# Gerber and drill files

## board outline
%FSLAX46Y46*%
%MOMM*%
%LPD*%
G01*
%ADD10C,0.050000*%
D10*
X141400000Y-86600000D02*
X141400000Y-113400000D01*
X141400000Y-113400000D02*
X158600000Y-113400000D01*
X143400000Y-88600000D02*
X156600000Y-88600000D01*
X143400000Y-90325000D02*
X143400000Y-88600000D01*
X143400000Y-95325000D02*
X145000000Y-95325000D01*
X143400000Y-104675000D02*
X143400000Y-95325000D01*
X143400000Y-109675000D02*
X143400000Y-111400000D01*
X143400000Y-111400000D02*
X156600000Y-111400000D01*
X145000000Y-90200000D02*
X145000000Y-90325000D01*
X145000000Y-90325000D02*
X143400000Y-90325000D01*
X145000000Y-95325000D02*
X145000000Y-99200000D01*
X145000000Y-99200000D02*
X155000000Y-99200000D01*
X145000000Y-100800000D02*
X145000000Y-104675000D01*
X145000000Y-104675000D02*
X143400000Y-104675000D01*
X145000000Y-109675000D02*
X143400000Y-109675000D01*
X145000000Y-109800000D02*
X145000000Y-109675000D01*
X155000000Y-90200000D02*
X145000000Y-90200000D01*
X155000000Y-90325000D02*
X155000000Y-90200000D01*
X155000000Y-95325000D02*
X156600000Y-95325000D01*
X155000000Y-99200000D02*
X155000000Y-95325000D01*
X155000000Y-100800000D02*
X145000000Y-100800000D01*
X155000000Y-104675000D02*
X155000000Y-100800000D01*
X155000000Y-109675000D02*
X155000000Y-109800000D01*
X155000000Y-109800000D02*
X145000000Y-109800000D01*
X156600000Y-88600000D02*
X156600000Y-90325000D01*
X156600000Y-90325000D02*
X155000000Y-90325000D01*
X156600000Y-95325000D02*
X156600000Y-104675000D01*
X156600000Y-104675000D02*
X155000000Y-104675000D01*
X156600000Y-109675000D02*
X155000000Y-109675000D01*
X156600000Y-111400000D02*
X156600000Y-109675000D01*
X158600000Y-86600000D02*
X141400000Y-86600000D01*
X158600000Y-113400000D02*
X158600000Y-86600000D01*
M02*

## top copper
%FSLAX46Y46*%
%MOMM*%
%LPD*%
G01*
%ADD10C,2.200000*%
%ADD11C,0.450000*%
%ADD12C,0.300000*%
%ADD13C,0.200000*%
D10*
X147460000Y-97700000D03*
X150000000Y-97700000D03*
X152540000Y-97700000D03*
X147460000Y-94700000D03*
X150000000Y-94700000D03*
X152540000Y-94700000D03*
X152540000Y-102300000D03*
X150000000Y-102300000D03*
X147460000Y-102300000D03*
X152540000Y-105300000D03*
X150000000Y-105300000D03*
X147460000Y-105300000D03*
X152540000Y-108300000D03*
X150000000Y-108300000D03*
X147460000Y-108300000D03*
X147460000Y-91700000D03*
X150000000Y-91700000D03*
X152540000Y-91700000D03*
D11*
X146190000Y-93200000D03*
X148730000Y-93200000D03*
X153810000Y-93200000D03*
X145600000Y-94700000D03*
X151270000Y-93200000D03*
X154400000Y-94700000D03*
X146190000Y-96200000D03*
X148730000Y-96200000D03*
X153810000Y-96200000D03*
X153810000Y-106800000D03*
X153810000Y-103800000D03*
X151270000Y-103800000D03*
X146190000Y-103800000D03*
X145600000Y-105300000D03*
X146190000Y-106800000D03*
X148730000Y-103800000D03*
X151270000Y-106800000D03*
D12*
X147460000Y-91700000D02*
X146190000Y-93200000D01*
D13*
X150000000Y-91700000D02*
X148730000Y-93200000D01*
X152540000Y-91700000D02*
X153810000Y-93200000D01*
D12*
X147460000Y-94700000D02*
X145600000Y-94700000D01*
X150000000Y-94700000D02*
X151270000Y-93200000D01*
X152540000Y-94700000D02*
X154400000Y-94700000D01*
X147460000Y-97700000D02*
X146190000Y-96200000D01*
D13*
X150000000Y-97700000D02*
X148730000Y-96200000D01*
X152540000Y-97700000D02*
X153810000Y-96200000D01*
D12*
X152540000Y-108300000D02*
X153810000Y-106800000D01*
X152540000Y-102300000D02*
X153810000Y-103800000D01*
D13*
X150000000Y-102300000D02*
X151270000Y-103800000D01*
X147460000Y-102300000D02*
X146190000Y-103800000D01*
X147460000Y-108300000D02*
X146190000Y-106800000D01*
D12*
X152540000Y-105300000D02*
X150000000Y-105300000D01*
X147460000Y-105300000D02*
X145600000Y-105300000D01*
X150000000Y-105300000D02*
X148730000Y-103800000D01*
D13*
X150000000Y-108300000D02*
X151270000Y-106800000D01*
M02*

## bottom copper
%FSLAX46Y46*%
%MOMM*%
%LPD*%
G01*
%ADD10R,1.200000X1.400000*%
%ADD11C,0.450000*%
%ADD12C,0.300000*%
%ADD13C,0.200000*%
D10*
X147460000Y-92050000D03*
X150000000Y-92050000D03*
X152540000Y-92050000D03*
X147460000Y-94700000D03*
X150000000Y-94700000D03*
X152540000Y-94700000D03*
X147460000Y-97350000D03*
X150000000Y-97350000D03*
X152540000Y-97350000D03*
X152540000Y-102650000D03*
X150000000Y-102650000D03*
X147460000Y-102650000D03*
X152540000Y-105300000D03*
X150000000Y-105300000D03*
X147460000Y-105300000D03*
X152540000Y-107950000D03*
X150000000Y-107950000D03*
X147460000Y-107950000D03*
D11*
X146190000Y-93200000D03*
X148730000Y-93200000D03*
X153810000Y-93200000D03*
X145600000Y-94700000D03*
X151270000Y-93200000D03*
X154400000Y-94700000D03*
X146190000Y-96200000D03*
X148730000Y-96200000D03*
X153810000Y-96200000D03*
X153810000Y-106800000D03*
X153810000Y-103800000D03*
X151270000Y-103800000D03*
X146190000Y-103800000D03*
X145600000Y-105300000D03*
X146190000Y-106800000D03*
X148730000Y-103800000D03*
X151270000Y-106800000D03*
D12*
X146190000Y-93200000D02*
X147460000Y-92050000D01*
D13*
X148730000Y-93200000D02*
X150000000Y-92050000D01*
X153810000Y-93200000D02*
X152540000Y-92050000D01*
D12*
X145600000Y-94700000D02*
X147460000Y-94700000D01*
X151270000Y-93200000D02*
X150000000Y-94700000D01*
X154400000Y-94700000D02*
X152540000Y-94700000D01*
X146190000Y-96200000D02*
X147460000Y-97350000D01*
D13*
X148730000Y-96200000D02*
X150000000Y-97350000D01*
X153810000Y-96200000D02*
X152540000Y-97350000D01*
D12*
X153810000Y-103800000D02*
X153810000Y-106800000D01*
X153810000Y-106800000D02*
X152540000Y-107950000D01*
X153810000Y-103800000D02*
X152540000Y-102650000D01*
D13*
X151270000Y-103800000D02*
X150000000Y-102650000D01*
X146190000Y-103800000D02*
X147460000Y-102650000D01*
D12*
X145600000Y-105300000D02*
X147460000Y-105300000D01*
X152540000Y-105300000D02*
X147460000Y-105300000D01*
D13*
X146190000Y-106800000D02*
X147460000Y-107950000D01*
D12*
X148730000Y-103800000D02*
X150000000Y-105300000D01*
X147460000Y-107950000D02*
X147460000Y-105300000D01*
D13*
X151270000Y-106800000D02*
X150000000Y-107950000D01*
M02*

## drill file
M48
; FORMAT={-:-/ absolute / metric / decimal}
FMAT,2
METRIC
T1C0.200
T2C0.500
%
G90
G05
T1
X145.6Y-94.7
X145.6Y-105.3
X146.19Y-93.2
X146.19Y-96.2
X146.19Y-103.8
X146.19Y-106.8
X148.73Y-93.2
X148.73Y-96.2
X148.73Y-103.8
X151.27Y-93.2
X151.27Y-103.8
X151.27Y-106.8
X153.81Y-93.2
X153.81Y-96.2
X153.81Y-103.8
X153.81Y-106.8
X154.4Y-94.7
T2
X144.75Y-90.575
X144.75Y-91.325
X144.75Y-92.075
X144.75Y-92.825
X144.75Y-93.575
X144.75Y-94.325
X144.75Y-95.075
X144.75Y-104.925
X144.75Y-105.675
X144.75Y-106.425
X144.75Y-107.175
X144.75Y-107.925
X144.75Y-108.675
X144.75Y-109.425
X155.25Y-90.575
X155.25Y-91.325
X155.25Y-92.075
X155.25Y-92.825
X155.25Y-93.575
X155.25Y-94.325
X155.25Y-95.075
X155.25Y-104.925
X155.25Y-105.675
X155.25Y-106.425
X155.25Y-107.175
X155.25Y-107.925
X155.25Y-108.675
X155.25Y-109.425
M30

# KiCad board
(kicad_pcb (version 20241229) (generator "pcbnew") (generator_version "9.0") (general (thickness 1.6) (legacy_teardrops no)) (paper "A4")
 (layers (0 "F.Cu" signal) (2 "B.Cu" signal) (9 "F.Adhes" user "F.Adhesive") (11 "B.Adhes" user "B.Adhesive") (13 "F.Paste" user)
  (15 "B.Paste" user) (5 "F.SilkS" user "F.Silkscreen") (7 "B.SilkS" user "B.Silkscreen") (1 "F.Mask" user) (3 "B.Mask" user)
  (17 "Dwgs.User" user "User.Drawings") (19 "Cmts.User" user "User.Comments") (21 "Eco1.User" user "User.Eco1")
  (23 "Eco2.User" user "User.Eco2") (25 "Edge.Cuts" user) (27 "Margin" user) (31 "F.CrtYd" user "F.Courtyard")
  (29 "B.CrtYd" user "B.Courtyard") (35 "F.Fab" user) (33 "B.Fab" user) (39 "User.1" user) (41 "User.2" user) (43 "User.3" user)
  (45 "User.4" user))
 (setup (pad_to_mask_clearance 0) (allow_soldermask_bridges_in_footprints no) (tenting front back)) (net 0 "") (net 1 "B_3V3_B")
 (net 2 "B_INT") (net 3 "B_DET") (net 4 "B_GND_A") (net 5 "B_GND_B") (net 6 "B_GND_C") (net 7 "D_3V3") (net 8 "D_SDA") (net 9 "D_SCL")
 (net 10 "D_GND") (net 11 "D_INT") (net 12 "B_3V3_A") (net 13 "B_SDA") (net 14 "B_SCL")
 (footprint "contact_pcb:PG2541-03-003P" (layer "F.Cu") (at 150 97.7)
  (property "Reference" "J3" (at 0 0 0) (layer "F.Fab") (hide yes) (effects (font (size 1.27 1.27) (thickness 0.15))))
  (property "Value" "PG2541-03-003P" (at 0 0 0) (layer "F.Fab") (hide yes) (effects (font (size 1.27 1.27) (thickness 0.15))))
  (pad "1" smd circle (at -2.54 0) (size 2.2 2.2) (layers "F.Cu" "F.Mask" "F.Paste") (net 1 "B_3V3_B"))
  (pad "2" smd circle (at 0 0) (size 2.2 2.2) (layers "F.Cu" "F.Mask" "F.Paste") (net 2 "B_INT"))
  (pad "3" smd circle (at 2.54 0) (size 2.2 2.2) (layers "F.Cu" "F.Mask" "F.Paste") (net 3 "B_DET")))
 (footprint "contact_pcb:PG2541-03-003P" (layer "F.Cu") (at 150 94.7)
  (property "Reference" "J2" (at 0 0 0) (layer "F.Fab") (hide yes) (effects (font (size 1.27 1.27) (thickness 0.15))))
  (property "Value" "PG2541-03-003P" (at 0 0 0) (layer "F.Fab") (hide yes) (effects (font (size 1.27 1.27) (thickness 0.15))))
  (pad "1" smd circle (at -2.54 0) (size 2.2 2.2) (layers "F.Cu" "F.Mask" "F.Paste") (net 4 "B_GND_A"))
  (pad "2" smd circle (at 0 0) (size 2.2 2.2) (layers "F.Cu" "F.Mask" "F.Paste") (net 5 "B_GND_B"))
  (pad "3" smd circle (at 2.54 0) (size 2.2 2.2) (layers "F.Cu" "F.Mask" "F.Paste") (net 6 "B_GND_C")))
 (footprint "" (layer "F.Cu") (at 150 105.3)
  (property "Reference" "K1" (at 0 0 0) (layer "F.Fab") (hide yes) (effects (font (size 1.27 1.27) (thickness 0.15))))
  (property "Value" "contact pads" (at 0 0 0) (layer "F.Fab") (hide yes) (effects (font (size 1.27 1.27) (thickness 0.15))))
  (pad "1" smd circle (at 2.54 -3) (size 2.2 2.2) (layers "F.Cu" "F.Mask") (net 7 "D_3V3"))
  (pad "2" smd circle (at 0 -3) (size 2.2 2.2) (layers "F.Cu" "F.Mask") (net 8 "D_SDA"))
  (pad "3" smd circle (at -2.54 -3) (size 2.2 2.2) (layers "F.Cu" "F.Mask") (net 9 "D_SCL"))
  (pad "4" smd circle (at 2.54 0) (size 2.2 2.2) (layers "F.Cu" "F.Mask") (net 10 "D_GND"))
  (pad "5" smd circle (at 0 0) (size 2.2 2.2) (layers "F.Cu" "F.Mask") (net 10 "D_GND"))
  (pad "6" smd circle (at -2.54 0) (size 2.2 2.2) (layers "F.Cu" "F.Mask") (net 10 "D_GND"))
  (pad "7" smd circle (at 2.54 3) (size 2.2 2.2) (layers "F.Cu" "F.Mask") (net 7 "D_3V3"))
  (pad "8" smd circle (at 0 3) (size 2.2 2.2) (layers "F.Cu" "F.Mask") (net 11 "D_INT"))
  (pad "9" smd circle (at -2.54 3) (size 2.2 2.2) (layers "F.Cu" "F.Mask") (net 10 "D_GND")))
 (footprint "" (layer "F.Cu") (at 150 94.7)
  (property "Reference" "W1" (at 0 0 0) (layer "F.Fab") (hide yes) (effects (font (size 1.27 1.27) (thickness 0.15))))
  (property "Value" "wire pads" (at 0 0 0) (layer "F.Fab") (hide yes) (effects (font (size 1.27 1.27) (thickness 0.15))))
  (pad "1" smd rect (at -2.54 -2.65) (size 1.2 1.4) (layers "B.Cu" "B.Mask") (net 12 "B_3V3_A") (thermal_bridge_angle 45))
  (pad "2" smd rect (at 0 -2.65) (size 1.2 1.4) (layers "B.Cu" "B.Mask") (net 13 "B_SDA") (thermal_bridge_angle 45))
  (pad "3" smd rect (at 2.54 -2.65) (size 1.2 1.4) (layers "B.Cu" "B.Mask") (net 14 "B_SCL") (thermal_bridge_angle 45))
  (pad "4" smd rect (at -2.54 0) (size 1.2 1.4) (layers "B.Cu" "B.Mask") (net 4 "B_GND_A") (thermal_bridge_angle 45))
  (pad "5" smd rect (at 0 0) (size 1.2 1.4) (layers "B.Cu" "B.Mask") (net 5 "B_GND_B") (thermal_bridge_angle 45))
  (pad "6" smd rect (at 2.54 0) (size 1.2 1.4) (layers "B.Cu" "B.Mask") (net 6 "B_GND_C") (thermal_bridge_angle 45))
  (pad "7" smd rect (at -2.54 2.65) (size 1.2 1.4) (layers "B.Cu" "B.Mask") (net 1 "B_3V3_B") (thermal_bridge_angle 45))
  (pad "8" smd rect (at 0 2.65) (size 1.2 1.4) (layers "B.Cu" "B.Mask") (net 2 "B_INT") (thermal_bridge_angle 45))
  (pad "9" smd rect (at 2.54 2.65) (size 1.2 1.4) (layers "B.Cu" "B.Mask") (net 3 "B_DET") (thermal_bridge_angle 45)))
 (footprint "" (layer "F.Cu") (at 150 105.3)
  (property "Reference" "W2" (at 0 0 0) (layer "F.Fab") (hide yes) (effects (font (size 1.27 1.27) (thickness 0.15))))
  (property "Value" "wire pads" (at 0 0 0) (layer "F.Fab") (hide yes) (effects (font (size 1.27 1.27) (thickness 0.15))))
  (pad "1" smd rect (at 2.54 -2.65) (size 1.2 1.4) (layers "B.Cu" "B.Mask") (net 7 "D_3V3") (thermal_bridge_angle 45))
  (pad "2" smd rect (at 0 -2.65) (size 1.2 1.4) (layers "B.Cu" "B.Mask") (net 8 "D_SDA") (thermal_bridge_angle 45))
  (pad "3" smd rect (at -2.54 -2.65) (size 1.2 1.4) (layers "B.Cu" "B.Mask") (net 9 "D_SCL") (thermal_bridge_angle 45))
  (pad "4" smd rect (at 2.54 0) (size 1.2 1.4) (layers "B.Cu" "B.Mask") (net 10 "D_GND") (thermal_bridge_angle 45))
  (pad "5" smd rect (at 0 0) (size 1.2 1.4) (layers "B.Cu" "B.Mask") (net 10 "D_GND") (thermal_bridge_angle 45))
  (pad "6" smd rect (at -2.54 0) (size 1.2 1.4) (layers "B.Cu" "B.Mask") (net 10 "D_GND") (thermal_bridge_angle 45))
  (pad "7" smd rect (at 2.54 2.65) (size 1.2 1.4) (layers "B.Cu" "B.Mask") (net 7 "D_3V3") (thermal_bridge_angle 45))
  (pad "8" smd rect (at 0 2.65) (size 1.2 1.4) (layers "B.Cu" "B.Mask") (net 11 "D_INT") (thermal_bridge_angle 45))
  (pad "9" smd rect (at -2.54 2.65) (size 1.2 1.4) (layers "B.Cu" "B.Mask") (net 10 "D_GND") (thermal_bridge_angle 45)))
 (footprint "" (layer "F.Cu") (at 150 100)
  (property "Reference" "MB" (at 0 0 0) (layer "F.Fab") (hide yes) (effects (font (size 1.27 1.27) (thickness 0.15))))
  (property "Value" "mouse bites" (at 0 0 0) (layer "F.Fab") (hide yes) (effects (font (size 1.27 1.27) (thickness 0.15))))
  (pad "" np_thru_hole circle (at -5.25 -9.425) (size 0.5 0.5) (drill 0.5) (layers "*.Mask"))
  (pad "" np_thru_hole circle (at -5.25 -8.675) (size 0.5 0.5) (drill 0.5) (layers "*.Mask"))
  (pad "" np_thru_hole circle (at -5.25 -7.925) (size 0.5 0.5) (drill 0.5) (layers "*.Mask"))
  (pad "" np_thru_hole circle (at -5.25 -7.175) (size 0.5 0.5) (drill 0.5) (layers "*.Mask"))
  (pad "" np_thru_hole circle (at -5.25 -6.425) (size 0.5 0.5) (drill 0.5) (layers "*.Mask"))
  (pad "" np_thru_hole circle (at -5.25 -5.675) (size 0.5 0.5) (drill 0.5) (layers "*.Mask"))
  (pad "" np_thru_hole circle (at -5.25 -4.925) (size 0.5 0.5) (drill 0.5) (layers "*.Mask"))
  (pad "" np_thru_hole circle (at -5.25 4.925) (size 0.5 0.5) (drill 0.5) (layers "*.Mask"))
  (pad "" np_thru_hole circle (at -5.25 5.675) (size 0.5 0.5) (drill 0.5) (layers "*.Mask"))
  (pad "" np_thru_hole circle (at -5.25 6.425) (size 0.5 0.5) (drill 0.5) (layers "*.Mask"))
  (pad "" np_thru_hole circle (at -5.25 7.175) (size 0.5 0.5) (drill 0.5) (layers "*.Mask"))
  (pad "" np_thru_hole circle (at -5.25 7.925) (size 0.5 0.5) (drill 0.5) (layers "*.Mask"))
  (pad "" np_thru_hole circle (at -5.25 8.675) (size 0.5 0.5) (drill 0.5) (layers "*.Mask"))
  (pad "" np_thru_hole circle (at -5.25 9.425) (size 0.5 0.5) (drill 0.5) (layers "*.Mask"))
  (pad "" np_thru_hole circle (at 5.25 -9.425) (size 0.5 0.5) (drill 0.5) (layers "*.Mask"))
  (pad "" np_thru_hole circle (at 5.25 -8.675) (size 0.5 0.5) (drill 0.5) (layers "*.Mask"))
  (pad "" np_thru_hole circle (at 5.25 -7.925) (size 0.5 0.5) (drill 0.5) (layers "*.Mask"))
  (pad "" np_thru_hole circle (at 5.25 -7.175) (size 0.5 0.5) (drill 0.5) (layers "*.Mask"))
  (pad "" np_thru_hole circle (at 5.25 -6.425) (size 0.5 0.5) (drill 0.5) (layers "*.Mask"))
  (pad "" np_thru_hole circle (at 5.25 -5.675) (size 0.5 0.5) (drill 0.5) (layers "*.Mask"))
  (pad "" np_thru_hole circle (at 5.25 -4.925) (size 0.5 0.5) (drill 0.5) (layers "*.Mask"))
  (pad "" np_thru_hole circle (at 5.25 4.925) (size 0.5 0.5) (drill 0.5) (layers "*.Mask"))
  (pad "" np_thru_hole circle (at 5.25 5.675) (size 0.5 0.5) (drill 0.5) (layers "*.Mask"))
  (pad "" np_thru_hole circle (at 5.25 6.425) (size 0.5 0.5) (drill 0.5) (layers "*.Mask"))
  (pad "" np_thru_hole circle (at 5.25 7.175) (size 0.5 0.5) (drill 0.5) (layers "*.Mask"))
  (pad "" np_thru_hole circle (at 5.25 7.925) (size 0.5 0.5) (drill 0.5) (layers "*.Mask"))
  (pad "" np_thru_hole circle (at 5.25 8.675) (size 0.5 0.5) (drill 0.5) (layers "*.Mask"))
  (pad "" np_thru_hole circle (at 5.25 9.425) (size 0.5 0.5) (drill 0.5) (layers "*.Mask")))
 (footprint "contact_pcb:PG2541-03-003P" (layer "F.Cu") (at 150 91.7)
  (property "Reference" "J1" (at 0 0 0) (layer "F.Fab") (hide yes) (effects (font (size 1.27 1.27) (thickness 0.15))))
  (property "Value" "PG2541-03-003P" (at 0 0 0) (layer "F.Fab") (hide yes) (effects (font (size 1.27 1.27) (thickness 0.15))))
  (pad "1" smd circle (at -2.54 0) (size 2.2 2.2) (layers "F.Cu" "F.Mask" "F.Paste") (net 12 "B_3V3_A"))
  (pad "2" smd circle (at 0 0) (size 2.2 2.2) (layers "F.Cu" "F.Mask" "F.Paste") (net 13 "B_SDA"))
  (pad "3" smd circle (at 2.54 0) (size 2.2 2.2) (layers "F.Cu" "F.Mask" "F.Paste") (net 14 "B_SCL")))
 (gr_line (start 141.4 86.6) (end 141.4 113.4) (stroke (width 0.05) (type default)) (layer "Edge.Cuts"))
 (gr_line (start 141.4 113.4) (end 158.6 113.4) (stroke (width 0.05) (type default)) (layer "Edge.Cuts"))
 (gr_line (start 143.4 88.6) (end 156.6 88.6) (stroke (width 0.05) (type default)) (layer "Edge.Cuts"))
 (gr_line (start 143.4 90.325) (end 143.4 88.6) (stroke (width 0.05) (type default)) (layer "Edge.Cuts"))
 (gr_line (start 143.4 95.325) (end 145 95.325) (stroke (width 0.05) (type default)) (layer "Edge.Cuts"))
 (gr_line (start 143.4 104.675) (end 143.4 95.325) (stroke (width 0.05) (type default)) (layer "Edge.Cuts"))
 (gr_line (start 143.4 109.675) (end 143.4 111.4) (stroke (width 0.05) (type default)) (layer "Edge.Cuts"))
 (gr_line (start 143.4 111.4) (end 156.6 111.4) (stroke (width 0.05) (type default)) (layer "Edge.Cuts"))
 (gr_line (start 145 90.2) (end 145 90.325) (stroke (width 0.05) (type default)) (layer "Edge.Cuts"))
 (gr_line (start 145 90.325) (end 143.4 90.325) (stroke (width 0.05) (type default)) (layer "Edge.Cuts"))
 (gr_line (start 145 95.325) (end 145 99.2) (stroke (width 0.05) (type default)) (layer "Edge.Cuts"))
 (gr_line (start 145 99.2) (end 155 99.2) (stroke (width 0.05) (type default)) (layer "Edge.Cuts"))
 (gr_line (start 145 100.8) (end 145 104.675) (stroke (width 0.05) (type default)) (layer "Edge.Cuts"))
 (gr_line (start 145 104.675) (end 143.4 104.675) (stroke (width 0.05) (type default)) (layer "Edge.Cuts"))
 (gr_line (start 145 109.675) (end 143.4 109.675) (stroke (width 0.05) (type default)) (layer "Edge.Cuts"))
 (gr_line (start 145 109.8) (end 145 109.675) (stroke (width 0.05) (type default)) (layer "Edge.Cuts"))
 (gr_line (start 155 90.2) (end 145 90.2) (stroke (width 0.05) (type default)) (layer "Edge.Cuts"))
 (gr_line (start 155 90.325) (end 155 90.2) (stroke (width 0.05) (type default)) (layer "Edge.Cuts"))
 (gr_line (start 155 95.325) (end 156.6 95.325) (stroke (width 0.05) (type default)) (layer "Edge.Cuts"))
 (gr_line (start 155 99.2) (end 155 95.325) (stroke (width 0.05) (type default)) (layer "Edge.Cuts"))
 (gr_line (start 155 100.8) (end 145 100.8) (stroke (width 0.05) (type default)) (layer "Edge.Cuts"))
 (gr_line (start 155 104.675) (end 155 100.8) (stroke (width 0.05) (type default)) (layer "Edge.Cuts"))
 (gr_line (start 155 109.675) (end 155 109.8) (stroke (width 0.05) (type default)) (layer "Edge.Cuts"))
 (gr_line (start 155 109.8) (end 145 109.8) (stroke (width 0.05) (type default)) (layer "Edge.Cuts"))
 (gr_line (start 156.6 88.6) (end 156.6 90.325) (stroke (width 0.05) (type default)) (layer "Edge.Cuts"))
 (gr_line (start 156.6 90.325) (end 155 90.325) (stroke (width 0.05) (type default)) (layer "Edge.Cuts"))
 (gr_line (start 156.6 95.325) (end 156.6 104.675) (stroke (width 0.05) (type default)) (layer "Edge.Cuts"))
 (gr_line (start 156.6 104.675) (end 155 104.675) (stroke (width 0.05) (type default)) (layer "Edge.Cuts"))
 (gr_line (start 156.6 109.675) (end 155 109.675) (stroke (width 0.05) (type default)) (layer "Edge.Cuts"))
 (gr_line (start 156.6 111.4) (end 156.6 109.675) (stroke (width 0.05) (type default)) (layer "Edge.Cuts"))
 (gr_line (start 158.6 86.6) (end 141.4 86.6) (stroke (width 0.05) (type default)) (layer "Edge.Cuts"))
 (gr_line (start 158.6 113.4) (end 158.6 86.6) (stroke (width 0.05) (type default)) (layer "Edge.Cuts"))
 (segment (start 147.46 91.7) (end 146.19 93.2) (width 0.3) (layer "F.Cu") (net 12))
 (via (at 146.19 93.2) (size 0.45) (drill 0.2) (layers "F.Cu" "B.Cu") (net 12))
 (segment (start 146.19 93.2) (end 147.46 92.05) (width 0.3) (layer "B.Cu") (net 12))
 (segment (start 150 91.7) (end 148.73 93.2) (width 0.2) (layer "F.Cu") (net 13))
 (via (at 148.73 93.2) (size 0.45) (drill 0.2) (layers "F.Cu" "B.Cu") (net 13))
 (segment (start 148.73 93.2) (end 150 92.05) (width 0.2) (layer "B.Cu") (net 13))
 (segment (start 152.54 91.7) (end 153.81 93.2) (width 0.2) (layer "F.Cu") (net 14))
 (via (at 153.81 93.2) (size 0.45) (drill 0.2) (layers "F.Cu" "B.Cu") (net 14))
 (segment (start 153.81 93.2) (end 152.54 92.05) (width 0.2) (layer "B.Cu") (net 14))
 (segment (start 147.46 94.7) (end 145.6 94.7) (width 0.3) (layer "F.Cu") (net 4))
 (via (at 145.6 94.7) (size 0.45) (drill 0.2) (layers "F.Cu" "B.Cu") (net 4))
 (segment (start 145.6 94.7) (end 147.46 94.7) (width 0.3) (layer "B.Cu") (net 4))
 (segment (start 150 94.7) (end 151.27 93.2) (width 0.3) (layer "F.Cu") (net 5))
 (via (at 151.27 93.2) (size 0.45) (drill 0.2) (layers "F.Cu" "B.Cu") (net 5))
 (segment (start 151.27 93.2) (end 150 94.7) (width 0.3) (layer "B.Cu") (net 5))
 (segment (start 152.54 94.7) (end 154.4 94.7) (width 0.3) (layer "F.Cu") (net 6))
 (via (at 154.4 94.7) (size 0.45) (drill 0.2) (layers "F.Cu" "B.Cu") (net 6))
 (segment (start 154.4 94.7) (end 152.54 94.7) (width 0.3) (layer "B.Cu") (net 6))
 (segment (start 147.46 97.7) (end 146.19 96.2) (width 0.3) (layer "F.Cu") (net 1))
 (via (at 146.19 96.2) (size 0.45) (drill 0.2) (layers "F.Cu" "B.Cu") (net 1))
 (segment (start 146.19 96.2) (end 147.46 97.35) (width 0.3) (layer "B.Cu") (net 1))
 (segment (start 150 97.7) (end 148.73 96.2) (width 0.2) (layer "F.Cu") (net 2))
 (via (at 148.73 96.2) (size 0.45) (drill 0.2) (layers "F.Cu" "B.Cu") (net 2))
 (segment (start 148.73 96.2) (end 150 97.35) (width 0.2) (layer "B.Cu") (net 2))
 (segment (start 152.54 97.7) (end 153.81 96.2) (width 0.2) (layer "F.Cu") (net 3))
 (via (at 153.81 96.2) (size 0.45) (drill 0.2) (layers "F.Cu" "B.Cu") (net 3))
 (segment (start 153.81 96.2) (end 152.54 97.35) (width 0.2) (layer "B.Cu") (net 3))
 (segment (start 152.54 108.3) (end 153.81 106.8) (width 0.3) (layer "F.Cu") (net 7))
 (segment (start 152.54 102.3) (end 153.81 103.8) (width 0.3) (layer "F.Cu") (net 7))
 (via (at 153.81 106.8) (size 0.45) (drill 0.2) (layers "F.Cu" "B.Cu") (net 7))
 (via (at 153.81 103.8) (size 0.45) (drill 0.2) (layers "F.Cu" "B.Cu") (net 7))
 (segment (start 153.81 103.8) (end 153.81 106.8) (width 0.3) (layer "B.Cu") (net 7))
 (segment (start 153.81 106.8) (end 152.54 107.95) (width 0.3) (layer "B.Cu") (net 7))
 (segment (start 153.81 103.8) (end 152.54 102.65) (width 0.3) (layer "B.Cu") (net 7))
 (segment (start 150 102.3) (end 151.27 103.8) (width 0.2) (layer "F.Cu") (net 8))
 (via (at 151.27 103.8) (size 0.45) (drill 0.2) (layers "F.Cu" "B.Cu") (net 8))
 (segment (start 151.27 103.8) (end 150 102.65) (width 0.2) (layer "B.Cu") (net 8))
 (segment (start 147.46 102.3) (end 146.19 103.8) (width 0.2) (layer "F.Cu") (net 9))
 (via (at 146.19 103.8) (size 0.45) (drill 0.2) (layers "F.Cu" "B.Cu") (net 9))
 (segment (start 146.19 103.8) (end 147.46 102.65) (width 0.2) (layer "B.Cu") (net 9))
 (segment (start 147.46 108.3) (end 146.19 106.8) (width 0.2) (layer "F.Cu") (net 10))
 (segment (start 152.54 105.3) (end 150 105.3) (width 0.3) (layer "F.Cu") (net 10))
 (segment (start 147.46 105.3) (end 145.6 105.3) (width 0.3) (layer "F.Cu") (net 10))
 (segment (start 150 105.3) (end 148.73 103.8) (width 0.3) (layer "F.Cu") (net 10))
 (via (at 145.6 105.3) (size 0.45) (drill 0.2) (layers "F.Cu" "B.Cu") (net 10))
 (via (at 146.19 106.8) (size 0.45) (drill 0.2) (layers "F.Cu" "B.Cu") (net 10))
 (via (at 148.73 103.8) (size 0.45) (drill 0.2) (layers "F.Cu" "B.Cu") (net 10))
 (segment (start 145.6 105.3) (end 147.46 105.3) (width 0.3) (layer "B.Cu") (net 10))
 (segment (start 152.54 105.3) (end 147.46 105.3) (width 0.3) (layer "B.Cu") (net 10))
 (segment (start 146.19 106.8) (end 147.46 107.95) (width 0.2) (layer "B.Cu") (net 10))
 (segment (start 148.73 103.8) (end 150 105.3) (width 0.3) (layer "B.Cu") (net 10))
 (segment (start 147.46 107.95) (end 147.46 105.3) (width 0.3) (layer "B.Cu") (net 10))
 (segment (start 150 108.3) (end 151.27 106.8) (width 0.2) (layer "F.Cu") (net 11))
 (via (at 151.27 106.8) (size 0.45) (drill 0.2) (layers "F.Cu" "B.Cu") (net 11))
 (segment (start 151.27 106.8) (end 150 107.95) (width 0.2) (layer "B.Cu") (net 11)))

